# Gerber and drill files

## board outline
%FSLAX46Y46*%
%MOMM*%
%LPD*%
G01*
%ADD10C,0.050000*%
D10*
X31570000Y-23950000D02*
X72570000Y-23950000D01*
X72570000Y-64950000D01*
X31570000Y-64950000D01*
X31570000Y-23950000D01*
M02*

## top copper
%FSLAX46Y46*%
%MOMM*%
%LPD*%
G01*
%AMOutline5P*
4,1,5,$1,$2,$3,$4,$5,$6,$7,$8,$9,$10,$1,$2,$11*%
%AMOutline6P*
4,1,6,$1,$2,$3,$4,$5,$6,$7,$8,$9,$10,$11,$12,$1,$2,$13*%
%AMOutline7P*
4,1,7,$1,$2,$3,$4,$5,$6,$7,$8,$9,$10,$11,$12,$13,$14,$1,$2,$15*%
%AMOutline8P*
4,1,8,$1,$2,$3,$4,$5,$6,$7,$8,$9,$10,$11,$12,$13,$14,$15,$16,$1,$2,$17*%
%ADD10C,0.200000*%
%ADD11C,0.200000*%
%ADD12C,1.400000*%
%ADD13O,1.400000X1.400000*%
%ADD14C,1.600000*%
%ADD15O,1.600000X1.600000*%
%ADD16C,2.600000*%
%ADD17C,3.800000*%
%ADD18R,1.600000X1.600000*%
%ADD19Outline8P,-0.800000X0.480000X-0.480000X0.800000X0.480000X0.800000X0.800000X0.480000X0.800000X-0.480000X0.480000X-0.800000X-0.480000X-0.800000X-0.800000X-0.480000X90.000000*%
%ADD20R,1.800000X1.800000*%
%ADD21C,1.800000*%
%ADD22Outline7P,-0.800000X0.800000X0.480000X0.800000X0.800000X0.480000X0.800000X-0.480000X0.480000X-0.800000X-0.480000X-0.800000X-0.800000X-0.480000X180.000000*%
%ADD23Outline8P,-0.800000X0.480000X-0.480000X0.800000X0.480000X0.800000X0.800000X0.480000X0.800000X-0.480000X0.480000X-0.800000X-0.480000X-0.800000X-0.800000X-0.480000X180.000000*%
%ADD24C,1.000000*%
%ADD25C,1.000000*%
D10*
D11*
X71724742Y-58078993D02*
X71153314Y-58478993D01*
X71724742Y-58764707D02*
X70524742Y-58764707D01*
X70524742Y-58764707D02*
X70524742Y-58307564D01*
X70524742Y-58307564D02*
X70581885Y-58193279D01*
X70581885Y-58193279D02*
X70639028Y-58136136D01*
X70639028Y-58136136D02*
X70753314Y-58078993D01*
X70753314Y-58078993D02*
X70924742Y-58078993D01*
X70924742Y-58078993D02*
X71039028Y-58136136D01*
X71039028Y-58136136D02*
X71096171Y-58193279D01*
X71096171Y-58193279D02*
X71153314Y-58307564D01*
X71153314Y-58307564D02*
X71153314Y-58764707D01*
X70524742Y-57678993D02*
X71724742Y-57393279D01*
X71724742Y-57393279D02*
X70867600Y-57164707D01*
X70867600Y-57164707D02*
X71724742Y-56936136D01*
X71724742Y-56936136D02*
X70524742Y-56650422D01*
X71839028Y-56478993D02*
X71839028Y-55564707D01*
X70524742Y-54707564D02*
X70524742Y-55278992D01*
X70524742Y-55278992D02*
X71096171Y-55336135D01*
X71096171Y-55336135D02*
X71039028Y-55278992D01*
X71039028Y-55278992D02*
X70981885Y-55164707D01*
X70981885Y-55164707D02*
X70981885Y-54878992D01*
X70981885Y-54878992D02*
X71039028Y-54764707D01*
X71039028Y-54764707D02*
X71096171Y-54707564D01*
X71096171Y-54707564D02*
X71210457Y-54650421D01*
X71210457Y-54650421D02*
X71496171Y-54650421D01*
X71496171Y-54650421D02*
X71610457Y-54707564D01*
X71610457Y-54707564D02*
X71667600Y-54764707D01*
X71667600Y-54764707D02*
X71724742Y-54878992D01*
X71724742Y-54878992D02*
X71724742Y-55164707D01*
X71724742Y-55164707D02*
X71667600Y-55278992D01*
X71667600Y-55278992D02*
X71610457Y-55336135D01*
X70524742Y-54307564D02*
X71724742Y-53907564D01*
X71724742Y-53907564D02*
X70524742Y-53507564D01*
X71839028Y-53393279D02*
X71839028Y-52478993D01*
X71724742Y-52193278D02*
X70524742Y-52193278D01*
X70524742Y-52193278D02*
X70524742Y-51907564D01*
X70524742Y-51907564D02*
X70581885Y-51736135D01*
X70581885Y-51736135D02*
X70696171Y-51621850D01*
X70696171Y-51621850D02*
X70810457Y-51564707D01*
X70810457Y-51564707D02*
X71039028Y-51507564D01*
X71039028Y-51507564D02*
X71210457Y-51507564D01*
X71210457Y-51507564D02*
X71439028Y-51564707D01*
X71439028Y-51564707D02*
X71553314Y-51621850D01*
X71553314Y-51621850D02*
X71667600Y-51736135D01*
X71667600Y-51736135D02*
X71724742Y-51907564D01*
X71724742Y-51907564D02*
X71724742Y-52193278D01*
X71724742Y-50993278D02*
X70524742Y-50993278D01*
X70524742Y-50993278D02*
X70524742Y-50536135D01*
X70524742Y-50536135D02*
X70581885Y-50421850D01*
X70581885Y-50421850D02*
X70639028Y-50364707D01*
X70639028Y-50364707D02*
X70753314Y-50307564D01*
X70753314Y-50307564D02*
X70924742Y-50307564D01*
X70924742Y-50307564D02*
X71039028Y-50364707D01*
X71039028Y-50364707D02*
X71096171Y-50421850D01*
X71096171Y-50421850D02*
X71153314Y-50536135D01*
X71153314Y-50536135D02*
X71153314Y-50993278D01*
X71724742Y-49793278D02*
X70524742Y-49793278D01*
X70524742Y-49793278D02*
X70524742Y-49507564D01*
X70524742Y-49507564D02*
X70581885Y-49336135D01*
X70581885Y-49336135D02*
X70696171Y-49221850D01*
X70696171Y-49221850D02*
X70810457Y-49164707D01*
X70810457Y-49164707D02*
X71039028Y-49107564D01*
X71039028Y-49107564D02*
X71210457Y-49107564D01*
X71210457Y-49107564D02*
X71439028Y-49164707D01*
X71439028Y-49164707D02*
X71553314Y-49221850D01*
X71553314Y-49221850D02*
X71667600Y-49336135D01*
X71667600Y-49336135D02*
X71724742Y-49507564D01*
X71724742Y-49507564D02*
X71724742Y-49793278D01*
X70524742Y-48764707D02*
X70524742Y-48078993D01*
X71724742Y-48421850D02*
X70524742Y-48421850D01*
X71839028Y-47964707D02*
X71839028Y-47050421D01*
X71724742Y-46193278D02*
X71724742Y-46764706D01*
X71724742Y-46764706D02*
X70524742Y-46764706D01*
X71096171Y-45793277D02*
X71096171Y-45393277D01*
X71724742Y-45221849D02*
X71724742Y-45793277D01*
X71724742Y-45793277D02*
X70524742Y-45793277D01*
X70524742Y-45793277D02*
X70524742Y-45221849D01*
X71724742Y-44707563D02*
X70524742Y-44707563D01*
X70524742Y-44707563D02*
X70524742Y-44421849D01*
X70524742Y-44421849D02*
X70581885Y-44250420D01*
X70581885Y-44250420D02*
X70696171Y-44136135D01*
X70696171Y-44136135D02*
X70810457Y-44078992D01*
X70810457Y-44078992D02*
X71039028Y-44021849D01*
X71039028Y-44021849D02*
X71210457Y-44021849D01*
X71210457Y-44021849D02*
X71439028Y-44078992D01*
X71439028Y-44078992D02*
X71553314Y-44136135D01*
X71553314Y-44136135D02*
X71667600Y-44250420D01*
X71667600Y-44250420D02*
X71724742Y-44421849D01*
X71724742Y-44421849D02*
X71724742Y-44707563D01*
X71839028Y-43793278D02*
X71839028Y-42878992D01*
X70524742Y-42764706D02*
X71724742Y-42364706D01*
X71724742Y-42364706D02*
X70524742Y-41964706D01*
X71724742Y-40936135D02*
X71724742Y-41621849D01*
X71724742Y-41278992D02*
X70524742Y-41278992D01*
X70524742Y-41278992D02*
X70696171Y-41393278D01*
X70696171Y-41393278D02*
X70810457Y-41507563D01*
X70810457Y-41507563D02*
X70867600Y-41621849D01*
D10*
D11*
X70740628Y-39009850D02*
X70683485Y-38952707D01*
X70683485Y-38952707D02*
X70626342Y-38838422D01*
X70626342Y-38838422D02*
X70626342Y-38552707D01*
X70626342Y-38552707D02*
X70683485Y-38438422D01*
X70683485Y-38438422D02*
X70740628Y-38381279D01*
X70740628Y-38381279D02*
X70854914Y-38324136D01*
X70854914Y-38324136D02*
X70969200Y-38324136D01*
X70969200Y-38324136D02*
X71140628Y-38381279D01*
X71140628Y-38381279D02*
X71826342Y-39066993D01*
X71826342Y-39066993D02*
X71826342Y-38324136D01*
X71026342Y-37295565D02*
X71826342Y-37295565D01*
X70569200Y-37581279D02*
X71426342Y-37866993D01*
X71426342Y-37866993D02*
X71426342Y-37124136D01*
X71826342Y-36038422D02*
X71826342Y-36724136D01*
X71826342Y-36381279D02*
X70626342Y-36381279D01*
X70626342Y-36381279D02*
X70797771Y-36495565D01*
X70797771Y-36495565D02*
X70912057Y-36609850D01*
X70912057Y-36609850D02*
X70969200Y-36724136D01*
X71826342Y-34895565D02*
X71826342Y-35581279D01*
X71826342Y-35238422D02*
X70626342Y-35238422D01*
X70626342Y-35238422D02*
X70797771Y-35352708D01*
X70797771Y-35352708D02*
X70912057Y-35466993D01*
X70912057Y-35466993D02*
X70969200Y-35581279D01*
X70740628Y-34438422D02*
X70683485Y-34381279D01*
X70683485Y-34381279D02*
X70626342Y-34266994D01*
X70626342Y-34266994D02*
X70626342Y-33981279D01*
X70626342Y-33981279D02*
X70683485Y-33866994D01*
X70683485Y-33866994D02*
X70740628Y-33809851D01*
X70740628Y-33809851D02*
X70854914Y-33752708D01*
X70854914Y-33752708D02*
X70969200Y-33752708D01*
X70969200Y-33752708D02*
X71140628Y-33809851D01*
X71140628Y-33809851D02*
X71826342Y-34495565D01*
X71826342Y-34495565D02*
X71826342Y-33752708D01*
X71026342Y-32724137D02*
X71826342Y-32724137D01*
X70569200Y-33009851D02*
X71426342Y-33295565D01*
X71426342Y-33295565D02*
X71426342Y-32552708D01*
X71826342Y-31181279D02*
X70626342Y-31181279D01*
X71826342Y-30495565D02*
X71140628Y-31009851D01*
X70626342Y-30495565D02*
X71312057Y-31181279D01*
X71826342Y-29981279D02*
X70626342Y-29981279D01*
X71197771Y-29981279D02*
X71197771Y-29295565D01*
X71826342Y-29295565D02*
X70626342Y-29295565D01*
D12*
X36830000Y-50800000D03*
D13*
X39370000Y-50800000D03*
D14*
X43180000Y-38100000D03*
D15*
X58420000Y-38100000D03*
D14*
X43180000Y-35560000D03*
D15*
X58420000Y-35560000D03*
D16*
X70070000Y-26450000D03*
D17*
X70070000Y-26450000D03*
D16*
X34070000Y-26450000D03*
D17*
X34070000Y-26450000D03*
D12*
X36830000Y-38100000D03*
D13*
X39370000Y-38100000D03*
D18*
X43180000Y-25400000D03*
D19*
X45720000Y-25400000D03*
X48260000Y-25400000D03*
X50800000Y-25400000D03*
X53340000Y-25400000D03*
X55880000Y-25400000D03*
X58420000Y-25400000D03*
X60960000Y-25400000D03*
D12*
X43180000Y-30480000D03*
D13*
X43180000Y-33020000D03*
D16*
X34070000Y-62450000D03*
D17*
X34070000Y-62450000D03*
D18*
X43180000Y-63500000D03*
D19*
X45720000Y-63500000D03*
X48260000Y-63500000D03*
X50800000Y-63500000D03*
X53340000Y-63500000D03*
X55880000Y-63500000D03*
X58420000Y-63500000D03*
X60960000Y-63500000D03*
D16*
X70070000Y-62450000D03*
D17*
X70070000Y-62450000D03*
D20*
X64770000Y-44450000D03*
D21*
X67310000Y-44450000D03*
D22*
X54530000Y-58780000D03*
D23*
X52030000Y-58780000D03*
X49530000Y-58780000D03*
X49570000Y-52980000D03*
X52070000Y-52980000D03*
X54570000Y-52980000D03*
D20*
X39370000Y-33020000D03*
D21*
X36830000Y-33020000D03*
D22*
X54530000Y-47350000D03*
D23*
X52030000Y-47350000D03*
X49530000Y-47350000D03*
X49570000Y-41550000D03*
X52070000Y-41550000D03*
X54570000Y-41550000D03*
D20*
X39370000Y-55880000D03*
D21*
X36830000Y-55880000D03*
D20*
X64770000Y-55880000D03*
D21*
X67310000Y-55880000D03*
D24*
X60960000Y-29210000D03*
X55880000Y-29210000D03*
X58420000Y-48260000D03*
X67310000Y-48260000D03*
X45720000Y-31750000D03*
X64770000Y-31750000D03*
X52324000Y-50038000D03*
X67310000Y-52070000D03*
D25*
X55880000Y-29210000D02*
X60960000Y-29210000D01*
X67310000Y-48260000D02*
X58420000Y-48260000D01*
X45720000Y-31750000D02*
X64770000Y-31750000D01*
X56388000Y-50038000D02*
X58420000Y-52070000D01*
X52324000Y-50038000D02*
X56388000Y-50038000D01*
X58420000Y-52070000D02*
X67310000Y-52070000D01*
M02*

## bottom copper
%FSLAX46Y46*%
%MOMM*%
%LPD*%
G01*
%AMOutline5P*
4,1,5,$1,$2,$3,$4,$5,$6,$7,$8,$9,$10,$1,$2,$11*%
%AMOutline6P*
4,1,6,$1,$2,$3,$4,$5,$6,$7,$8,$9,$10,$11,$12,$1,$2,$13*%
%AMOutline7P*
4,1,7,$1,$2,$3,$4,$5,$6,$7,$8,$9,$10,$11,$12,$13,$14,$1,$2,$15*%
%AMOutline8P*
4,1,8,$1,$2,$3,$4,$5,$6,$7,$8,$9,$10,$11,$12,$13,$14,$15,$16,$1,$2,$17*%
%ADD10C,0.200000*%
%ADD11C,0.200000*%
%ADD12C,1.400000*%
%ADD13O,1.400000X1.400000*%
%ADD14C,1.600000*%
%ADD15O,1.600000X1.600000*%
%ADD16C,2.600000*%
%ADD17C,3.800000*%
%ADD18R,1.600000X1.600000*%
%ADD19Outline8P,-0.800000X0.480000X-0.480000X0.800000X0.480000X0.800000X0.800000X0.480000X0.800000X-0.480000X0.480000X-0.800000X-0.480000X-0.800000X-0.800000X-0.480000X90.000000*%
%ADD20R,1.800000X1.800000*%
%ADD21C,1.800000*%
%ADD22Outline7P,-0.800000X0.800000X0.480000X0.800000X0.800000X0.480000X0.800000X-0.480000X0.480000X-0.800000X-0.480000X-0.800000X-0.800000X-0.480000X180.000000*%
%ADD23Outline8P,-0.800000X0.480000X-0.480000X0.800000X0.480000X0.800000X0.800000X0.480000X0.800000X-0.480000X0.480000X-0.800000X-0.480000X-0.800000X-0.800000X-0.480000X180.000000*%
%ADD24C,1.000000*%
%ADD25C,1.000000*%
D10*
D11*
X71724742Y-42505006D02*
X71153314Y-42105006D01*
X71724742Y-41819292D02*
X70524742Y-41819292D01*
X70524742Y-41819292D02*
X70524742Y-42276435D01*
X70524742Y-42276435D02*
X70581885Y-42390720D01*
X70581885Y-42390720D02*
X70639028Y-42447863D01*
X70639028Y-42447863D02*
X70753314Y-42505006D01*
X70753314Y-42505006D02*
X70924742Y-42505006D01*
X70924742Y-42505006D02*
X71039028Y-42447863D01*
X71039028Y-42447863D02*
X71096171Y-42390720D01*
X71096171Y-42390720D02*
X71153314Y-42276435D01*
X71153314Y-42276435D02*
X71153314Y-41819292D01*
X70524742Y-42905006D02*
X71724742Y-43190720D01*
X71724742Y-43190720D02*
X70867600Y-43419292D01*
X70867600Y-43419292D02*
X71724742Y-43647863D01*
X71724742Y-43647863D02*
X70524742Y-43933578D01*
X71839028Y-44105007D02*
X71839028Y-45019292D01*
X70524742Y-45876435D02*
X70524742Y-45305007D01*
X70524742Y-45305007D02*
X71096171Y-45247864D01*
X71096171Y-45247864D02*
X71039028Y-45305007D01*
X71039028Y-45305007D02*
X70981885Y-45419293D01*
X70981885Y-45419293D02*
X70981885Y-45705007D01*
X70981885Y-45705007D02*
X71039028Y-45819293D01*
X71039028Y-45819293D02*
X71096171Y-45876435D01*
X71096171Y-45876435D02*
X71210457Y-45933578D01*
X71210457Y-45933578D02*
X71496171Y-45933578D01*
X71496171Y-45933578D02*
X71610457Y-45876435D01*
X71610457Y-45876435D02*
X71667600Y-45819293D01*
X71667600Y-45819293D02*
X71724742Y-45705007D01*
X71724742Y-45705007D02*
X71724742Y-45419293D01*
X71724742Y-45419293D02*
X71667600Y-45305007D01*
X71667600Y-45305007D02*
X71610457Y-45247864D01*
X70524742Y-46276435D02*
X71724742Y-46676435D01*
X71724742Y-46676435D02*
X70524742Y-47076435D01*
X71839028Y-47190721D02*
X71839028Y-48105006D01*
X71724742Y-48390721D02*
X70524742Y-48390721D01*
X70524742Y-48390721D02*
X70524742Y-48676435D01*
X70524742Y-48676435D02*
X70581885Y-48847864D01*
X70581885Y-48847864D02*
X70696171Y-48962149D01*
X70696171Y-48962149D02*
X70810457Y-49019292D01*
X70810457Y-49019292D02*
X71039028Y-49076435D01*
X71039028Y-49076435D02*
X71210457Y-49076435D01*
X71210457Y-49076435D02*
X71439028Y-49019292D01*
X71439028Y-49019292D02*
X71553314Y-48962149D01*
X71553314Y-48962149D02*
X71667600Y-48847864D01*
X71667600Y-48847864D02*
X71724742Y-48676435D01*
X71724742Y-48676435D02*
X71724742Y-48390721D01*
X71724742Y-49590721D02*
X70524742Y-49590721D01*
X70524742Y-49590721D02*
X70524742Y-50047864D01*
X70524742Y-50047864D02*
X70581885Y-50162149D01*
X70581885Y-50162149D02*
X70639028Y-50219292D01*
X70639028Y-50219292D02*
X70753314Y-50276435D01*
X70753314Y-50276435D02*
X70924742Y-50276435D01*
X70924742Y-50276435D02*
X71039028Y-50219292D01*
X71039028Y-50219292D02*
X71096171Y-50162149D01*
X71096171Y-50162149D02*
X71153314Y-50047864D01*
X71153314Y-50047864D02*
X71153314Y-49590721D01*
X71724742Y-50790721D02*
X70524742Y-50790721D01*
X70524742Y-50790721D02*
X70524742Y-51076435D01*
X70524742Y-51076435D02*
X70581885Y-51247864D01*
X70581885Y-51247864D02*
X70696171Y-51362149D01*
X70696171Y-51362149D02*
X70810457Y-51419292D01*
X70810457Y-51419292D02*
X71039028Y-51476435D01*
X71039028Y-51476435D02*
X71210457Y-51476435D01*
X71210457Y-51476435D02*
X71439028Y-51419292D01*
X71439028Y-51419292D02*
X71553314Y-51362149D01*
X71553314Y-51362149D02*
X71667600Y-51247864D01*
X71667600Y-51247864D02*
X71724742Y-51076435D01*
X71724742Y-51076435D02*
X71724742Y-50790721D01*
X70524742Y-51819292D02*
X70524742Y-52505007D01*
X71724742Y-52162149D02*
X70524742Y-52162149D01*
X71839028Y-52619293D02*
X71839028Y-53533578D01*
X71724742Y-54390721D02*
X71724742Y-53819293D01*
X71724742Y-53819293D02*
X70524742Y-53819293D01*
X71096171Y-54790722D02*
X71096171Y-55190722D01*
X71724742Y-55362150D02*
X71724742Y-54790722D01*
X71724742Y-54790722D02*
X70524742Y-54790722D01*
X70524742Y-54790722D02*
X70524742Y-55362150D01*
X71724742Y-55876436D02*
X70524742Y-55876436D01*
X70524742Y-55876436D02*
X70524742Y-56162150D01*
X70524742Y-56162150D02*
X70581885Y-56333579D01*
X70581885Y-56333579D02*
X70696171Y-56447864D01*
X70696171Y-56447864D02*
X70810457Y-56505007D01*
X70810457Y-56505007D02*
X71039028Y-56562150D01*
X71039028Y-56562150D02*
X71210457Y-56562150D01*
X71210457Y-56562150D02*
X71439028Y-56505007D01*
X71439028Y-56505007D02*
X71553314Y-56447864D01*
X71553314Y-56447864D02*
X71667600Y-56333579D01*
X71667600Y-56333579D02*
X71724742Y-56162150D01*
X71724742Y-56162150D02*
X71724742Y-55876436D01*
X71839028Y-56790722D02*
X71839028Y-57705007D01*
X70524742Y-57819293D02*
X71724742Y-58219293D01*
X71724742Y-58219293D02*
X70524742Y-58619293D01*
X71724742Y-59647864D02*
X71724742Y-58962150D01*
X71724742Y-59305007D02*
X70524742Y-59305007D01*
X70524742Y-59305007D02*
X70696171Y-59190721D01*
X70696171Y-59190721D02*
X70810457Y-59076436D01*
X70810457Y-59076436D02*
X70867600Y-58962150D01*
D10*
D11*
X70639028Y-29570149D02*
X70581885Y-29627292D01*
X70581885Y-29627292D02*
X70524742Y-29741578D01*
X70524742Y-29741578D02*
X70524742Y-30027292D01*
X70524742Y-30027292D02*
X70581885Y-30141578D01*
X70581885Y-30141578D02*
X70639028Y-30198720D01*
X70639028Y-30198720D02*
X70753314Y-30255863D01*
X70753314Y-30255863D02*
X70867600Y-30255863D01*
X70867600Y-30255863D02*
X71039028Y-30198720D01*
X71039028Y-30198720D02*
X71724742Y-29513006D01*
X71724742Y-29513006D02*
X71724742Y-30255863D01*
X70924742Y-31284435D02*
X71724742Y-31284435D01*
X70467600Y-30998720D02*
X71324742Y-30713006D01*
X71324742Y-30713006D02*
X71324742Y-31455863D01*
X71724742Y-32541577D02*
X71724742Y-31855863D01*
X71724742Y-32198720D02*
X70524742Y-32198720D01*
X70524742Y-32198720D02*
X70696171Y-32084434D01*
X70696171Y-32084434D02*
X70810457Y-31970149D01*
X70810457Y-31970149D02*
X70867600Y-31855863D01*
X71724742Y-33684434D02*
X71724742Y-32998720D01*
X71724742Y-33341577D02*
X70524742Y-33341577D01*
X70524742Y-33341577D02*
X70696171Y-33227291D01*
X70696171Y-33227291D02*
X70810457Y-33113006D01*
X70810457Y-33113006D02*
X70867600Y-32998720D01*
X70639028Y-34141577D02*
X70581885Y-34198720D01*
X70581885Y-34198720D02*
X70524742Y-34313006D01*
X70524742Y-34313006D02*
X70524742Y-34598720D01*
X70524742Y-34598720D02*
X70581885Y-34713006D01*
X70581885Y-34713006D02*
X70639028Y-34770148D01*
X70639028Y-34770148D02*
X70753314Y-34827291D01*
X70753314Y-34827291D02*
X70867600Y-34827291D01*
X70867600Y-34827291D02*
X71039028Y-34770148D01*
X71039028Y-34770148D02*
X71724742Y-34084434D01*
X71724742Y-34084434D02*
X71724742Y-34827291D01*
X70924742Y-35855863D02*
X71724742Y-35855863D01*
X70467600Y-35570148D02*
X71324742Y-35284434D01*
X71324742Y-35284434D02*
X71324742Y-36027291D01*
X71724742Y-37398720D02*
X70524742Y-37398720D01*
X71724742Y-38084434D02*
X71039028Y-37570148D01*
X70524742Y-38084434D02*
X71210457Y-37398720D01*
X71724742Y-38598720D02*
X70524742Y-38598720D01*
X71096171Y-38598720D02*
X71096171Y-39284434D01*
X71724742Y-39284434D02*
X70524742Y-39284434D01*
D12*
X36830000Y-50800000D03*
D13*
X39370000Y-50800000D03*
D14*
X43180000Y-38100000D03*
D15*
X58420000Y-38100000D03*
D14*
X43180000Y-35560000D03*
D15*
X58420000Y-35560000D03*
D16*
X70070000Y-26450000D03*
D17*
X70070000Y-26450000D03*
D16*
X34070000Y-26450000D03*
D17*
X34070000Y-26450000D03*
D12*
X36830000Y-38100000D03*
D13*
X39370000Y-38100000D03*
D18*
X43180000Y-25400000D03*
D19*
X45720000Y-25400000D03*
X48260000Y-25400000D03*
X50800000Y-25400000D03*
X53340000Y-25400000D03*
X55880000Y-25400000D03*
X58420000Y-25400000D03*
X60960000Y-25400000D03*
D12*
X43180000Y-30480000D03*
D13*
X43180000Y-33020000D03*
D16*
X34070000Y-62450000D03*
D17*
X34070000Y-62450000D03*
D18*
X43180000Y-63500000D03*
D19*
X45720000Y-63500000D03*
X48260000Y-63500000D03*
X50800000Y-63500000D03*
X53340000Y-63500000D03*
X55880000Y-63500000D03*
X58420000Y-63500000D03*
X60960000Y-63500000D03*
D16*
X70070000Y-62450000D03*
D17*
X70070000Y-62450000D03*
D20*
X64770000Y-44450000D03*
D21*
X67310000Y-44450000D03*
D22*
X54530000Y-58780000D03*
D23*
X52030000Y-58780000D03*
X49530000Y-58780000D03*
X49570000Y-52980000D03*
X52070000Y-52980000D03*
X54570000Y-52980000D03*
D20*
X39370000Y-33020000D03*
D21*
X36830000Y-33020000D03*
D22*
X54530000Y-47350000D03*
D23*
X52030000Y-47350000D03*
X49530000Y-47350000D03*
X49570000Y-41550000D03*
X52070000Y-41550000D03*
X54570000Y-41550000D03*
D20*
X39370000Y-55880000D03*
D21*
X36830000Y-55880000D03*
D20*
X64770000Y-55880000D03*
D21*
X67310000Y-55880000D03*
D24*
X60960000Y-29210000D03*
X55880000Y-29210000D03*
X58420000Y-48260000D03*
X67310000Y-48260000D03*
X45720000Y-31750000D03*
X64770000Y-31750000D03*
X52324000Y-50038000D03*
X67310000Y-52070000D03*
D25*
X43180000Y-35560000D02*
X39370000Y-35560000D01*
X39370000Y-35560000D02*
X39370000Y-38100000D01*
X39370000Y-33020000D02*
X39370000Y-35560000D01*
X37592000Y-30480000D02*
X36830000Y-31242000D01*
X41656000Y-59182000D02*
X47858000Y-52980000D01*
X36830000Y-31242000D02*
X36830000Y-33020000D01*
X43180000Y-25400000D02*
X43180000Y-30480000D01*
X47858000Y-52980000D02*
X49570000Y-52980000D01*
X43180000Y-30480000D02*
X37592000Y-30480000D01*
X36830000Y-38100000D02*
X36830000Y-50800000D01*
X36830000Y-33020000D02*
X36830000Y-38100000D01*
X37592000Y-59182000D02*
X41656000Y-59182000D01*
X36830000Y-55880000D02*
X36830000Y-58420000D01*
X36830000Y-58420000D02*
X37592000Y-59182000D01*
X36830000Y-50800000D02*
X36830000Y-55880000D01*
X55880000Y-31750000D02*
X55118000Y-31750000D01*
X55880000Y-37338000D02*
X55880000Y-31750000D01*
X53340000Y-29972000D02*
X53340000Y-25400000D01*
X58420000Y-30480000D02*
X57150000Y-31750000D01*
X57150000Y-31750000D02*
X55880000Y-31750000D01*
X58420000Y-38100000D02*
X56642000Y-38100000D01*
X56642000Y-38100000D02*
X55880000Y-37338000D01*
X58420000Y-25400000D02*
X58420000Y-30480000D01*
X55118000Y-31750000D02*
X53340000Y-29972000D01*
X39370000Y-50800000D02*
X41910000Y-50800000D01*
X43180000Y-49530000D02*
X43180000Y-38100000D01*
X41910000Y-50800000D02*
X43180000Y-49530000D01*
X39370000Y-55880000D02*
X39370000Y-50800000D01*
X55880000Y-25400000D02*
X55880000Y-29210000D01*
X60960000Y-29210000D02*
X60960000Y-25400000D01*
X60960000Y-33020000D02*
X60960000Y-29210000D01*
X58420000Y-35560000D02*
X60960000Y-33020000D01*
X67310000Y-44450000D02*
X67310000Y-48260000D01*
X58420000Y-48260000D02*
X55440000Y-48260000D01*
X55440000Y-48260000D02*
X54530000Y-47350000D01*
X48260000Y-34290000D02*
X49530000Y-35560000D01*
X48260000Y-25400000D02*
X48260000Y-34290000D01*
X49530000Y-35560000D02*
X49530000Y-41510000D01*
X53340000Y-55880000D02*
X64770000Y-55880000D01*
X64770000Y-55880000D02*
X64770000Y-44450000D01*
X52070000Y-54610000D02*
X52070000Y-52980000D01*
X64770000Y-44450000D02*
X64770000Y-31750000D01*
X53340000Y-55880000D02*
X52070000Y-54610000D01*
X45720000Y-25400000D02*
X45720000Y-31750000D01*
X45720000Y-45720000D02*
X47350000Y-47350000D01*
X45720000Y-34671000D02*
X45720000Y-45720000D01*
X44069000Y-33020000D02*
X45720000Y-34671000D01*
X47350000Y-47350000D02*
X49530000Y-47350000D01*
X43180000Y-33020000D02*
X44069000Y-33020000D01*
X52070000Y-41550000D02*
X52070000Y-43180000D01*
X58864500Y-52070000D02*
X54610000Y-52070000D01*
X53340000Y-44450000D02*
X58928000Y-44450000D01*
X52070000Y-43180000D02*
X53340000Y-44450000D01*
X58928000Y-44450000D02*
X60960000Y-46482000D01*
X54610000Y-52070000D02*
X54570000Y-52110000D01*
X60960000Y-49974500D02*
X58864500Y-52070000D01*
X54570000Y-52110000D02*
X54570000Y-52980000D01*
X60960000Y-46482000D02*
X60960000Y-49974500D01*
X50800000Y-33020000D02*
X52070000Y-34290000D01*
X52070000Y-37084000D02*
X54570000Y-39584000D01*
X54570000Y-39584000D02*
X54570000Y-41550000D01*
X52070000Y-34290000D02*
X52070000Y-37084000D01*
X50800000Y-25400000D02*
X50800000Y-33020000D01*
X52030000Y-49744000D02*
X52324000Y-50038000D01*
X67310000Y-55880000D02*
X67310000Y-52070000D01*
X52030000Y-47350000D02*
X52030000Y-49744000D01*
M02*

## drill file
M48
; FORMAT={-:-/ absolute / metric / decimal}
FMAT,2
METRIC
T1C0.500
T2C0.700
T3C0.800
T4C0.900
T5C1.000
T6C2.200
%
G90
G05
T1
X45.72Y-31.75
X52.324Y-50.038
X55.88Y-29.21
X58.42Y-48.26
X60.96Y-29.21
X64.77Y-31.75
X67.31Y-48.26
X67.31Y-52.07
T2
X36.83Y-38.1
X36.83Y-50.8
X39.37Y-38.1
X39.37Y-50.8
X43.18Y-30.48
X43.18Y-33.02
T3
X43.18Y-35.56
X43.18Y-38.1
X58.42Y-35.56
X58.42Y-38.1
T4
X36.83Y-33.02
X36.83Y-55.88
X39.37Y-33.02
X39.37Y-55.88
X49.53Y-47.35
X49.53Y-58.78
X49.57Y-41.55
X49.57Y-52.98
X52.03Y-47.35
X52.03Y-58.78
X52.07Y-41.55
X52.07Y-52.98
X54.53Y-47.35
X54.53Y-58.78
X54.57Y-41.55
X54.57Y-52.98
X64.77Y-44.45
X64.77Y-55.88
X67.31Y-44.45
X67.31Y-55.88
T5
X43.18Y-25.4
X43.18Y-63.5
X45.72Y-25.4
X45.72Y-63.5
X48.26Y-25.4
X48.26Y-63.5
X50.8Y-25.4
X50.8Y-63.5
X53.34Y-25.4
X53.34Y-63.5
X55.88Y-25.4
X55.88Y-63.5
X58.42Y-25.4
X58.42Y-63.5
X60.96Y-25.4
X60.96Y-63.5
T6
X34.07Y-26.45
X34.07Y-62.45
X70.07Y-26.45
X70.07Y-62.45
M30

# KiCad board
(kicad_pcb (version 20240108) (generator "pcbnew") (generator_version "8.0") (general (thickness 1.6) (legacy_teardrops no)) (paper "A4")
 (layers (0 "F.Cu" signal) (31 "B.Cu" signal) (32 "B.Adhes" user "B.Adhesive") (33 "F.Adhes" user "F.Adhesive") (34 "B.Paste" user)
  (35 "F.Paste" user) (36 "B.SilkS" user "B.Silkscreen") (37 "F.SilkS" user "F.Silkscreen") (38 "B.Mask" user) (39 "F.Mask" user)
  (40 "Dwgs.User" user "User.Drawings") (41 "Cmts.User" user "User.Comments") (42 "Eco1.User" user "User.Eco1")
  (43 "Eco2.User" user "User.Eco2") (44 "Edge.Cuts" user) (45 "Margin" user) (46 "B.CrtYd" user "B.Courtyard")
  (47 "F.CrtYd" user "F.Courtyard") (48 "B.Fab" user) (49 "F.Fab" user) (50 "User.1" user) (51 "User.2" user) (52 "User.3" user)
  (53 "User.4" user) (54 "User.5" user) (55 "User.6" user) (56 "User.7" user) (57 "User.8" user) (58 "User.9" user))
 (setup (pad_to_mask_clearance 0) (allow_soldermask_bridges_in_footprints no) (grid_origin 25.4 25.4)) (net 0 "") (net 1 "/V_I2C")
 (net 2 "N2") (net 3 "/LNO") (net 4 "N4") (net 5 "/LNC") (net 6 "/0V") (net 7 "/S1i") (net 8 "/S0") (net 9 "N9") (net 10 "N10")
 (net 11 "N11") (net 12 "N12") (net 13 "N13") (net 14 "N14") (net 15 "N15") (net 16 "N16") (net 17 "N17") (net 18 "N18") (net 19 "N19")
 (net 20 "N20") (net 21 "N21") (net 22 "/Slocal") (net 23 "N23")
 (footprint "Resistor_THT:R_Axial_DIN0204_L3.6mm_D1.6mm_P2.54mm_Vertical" (layer "F.Cu") (at 36.83 50.8)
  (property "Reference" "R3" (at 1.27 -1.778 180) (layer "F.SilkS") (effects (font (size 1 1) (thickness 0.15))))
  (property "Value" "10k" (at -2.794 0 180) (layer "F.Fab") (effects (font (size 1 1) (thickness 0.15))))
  (pad "1" thru_hole circle (at 0 0) (size 1.4 1.4) (drill 0.7) (layers "*.Cu" "*.Mask") (remove_unused_layers no) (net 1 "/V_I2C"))
  (pad "2" thru_hole oval (at 2.54 0) (size 1.4 1.4) (drill 0.7) (layers "*.Cu" "*.Mask") (remove_unused_layers no) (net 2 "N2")))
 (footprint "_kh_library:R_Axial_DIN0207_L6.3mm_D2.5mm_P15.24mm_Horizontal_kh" (layer "F.Cu") (at 43.18 38.1)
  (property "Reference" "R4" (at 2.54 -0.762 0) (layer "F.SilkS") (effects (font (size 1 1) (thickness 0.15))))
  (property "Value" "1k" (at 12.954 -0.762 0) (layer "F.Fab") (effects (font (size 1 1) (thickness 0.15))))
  (pad "1" thru_hole circle (at 0 0) (size 1.6 1.6) (drill 0.8) (layers "*.Cu" "*.Mask") (remove_unused_layers no) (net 2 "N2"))
  (pad "2" thru_hole oval (at 15.24 0) (size 1.6 1.6) (drill 0.8) (layers "*.Cu" "*.Mask") (remove_unused_layers no) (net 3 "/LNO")))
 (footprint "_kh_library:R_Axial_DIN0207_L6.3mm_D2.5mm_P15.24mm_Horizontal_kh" (layer "F.Cu") (at 43.18 35.56)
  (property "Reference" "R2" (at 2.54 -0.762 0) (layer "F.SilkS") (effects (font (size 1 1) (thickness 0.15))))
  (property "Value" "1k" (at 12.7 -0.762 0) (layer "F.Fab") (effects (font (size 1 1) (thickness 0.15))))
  (pad "1" thru_hole circle (at 0 0) (size 1.6 1.6) (drill 0.8) (layers "*.Cu" "*.Mask") (remove_unused_layers no) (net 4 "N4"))
  (pad "2" thru_hole oval (at 15.24 0) (size 1.6 1.6) (drill 0.8) (layers "*.Cu" "*.Mask") (remove_unused_layers no) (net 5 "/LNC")))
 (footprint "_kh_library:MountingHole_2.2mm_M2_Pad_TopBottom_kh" (layer "F.Cu") (at 70.07 26.45)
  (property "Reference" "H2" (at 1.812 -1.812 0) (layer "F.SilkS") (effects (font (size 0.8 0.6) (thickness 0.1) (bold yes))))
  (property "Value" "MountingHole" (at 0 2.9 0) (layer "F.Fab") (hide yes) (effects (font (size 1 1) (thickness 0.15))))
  (pad "1" thru_hole circle (at 0 0) (size 2.6 2.6) (drill 2.2) (layers "*.Cu" "*.Mask") (remove_unused_layers no))
  (pad "1" connect circle (at 0 0) (size 3.8 3.8) (layers "F.Cu" "F.Mask"))
  (pad "1" connect circle (at 0 0) (size 3.8 3.8) (layers "B.Cu" "B.Mask")))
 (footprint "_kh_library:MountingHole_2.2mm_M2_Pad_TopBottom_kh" (layer "F.Cu") (at 34.07 26.45)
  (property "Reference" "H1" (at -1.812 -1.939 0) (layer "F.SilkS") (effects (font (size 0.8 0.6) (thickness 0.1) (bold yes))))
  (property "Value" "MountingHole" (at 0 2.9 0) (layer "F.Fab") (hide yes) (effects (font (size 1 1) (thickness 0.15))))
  (pad "1" thru_hole circle (at 0 0) (size 2.6 2.6) (drill 2.2) (layers "*.Cu" "*.Mask") (remove_unused_layers no))
  (pad "1" connect circle (at 0 0) (size 3.8 3.8) (layers "F.Cu" "F.Mask"))
  (pad "1" connect circle (at 0 0) (size 3.8 3.8) (layers "B.Cu" "B.Mask")))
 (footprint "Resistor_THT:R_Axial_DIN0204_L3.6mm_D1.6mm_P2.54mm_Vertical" (layer "F.Cu") (at 36.83 38.1)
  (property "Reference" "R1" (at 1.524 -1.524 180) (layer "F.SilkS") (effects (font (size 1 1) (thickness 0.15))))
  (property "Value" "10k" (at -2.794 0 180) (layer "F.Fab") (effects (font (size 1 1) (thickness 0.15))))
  (pad "1" thru_hole circle (at 0 0) (size 1.4 1.4) (drill 0.7) (layers "*.Cu" "*.Mask") (remove_unused_layers no) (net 1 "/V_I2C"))
  (pad "2" thru_hole oval (at 2.54 0) (size 1.4 1.4) (drill 0.7) (layers "*.Cu" "*.Mask") (remove_unused_layers no) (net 4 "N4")))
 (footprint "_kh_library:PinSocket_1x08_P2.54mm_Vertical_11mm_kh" (layer "F.Cu") (at 43.18 25.4 90)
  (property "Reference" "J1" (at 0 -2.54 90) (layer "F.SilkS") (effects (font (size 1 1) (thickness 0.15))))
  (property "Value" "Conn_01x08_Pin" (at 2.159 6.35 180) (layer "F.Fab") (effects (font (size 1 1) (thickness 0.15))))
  (pad "1" thru_hole rect (at 0 0 90) (size 1.6 1.6) (drill 1) (layers "*.Cu" "*.Mask") (remove_unused_layers no) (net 1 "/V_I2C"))
  (pad "2" thru_hole roundrect (at 0 2.54 90) (size 1.6 1.6) (drill 1) (layers "*.Cu" "*.Mask") (remove_unused_layers no)
   (roundrect_rratio 0) (chamfer_ratio 0.2) (chamfer top_left top_right bottom_left bottom_right) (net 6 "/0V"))
  (pad "3" thru_hole roundrect (at 0 5.08 90) (size 1.6 1.6) (drill 1) (layers "*.Cu" "*.Mask") (remove_unused_layers no)
   (roundrect_rratio 0) (chamfer_ratio 0.2) (chamfer top_left top_right bottom_left bottom_right) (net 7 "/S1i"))
  (pad "4" thru_hole roundrect (at 0 7.62 90) (size 1.6 1.6) (drill 1) (layers "*.Cu" "*.Mask") (remove_unused_layers no)
   (roundrect_rratio 0) (chamfer_ratio 0.2) (chamfer top_left top_right bottom_left bottom_right) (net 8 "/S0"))
  (pad "5" thru_hole roundrect (at 0 10.16 90) (size 1.6 1.6) (drill 1) (layers "*.Cu" "*.Mask") (remove_unused_layers no)
   (roundrect_rratio 0) (chamfer_ratio 0.2) (chamfer top_left top_right bottom_left bottom_right) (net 3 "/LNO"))
  (pad "6" thru_hole roundrect (at 0 12.7 90) (size 1.6 1.6) (drill 1) (layers "*.Cu" "*.Mask") (remove_unused_layers no)
   (roundrect_rratio 0) (chamfer_ratio 0.2) (chamfer top_left top_right bottom_left bottom_right) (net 5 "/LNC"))
  (pad "7" thru_hole roundrect (at 0 15.24 90) (size 1.6 1.6) (drill 1) (layers "*.Cu" "*.Mask") (remove_unused_layers no)
   (roundrect_rratio 0) (chamfer_ratio 0.2) (chamfer top_left top_right bottom_left bottom_right) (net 3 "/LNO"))
  (pad "8" thru_hole roundrect (at 0 17.78 90) (size 1.6 1.6) (drill 1) (layers "*.Cu" "*.Mask") (remove_unused_layers no)
   (roundrect_rratio 0) (chamfer_ratio 0.2) (chamfer top_left top_right bottom_left bottom_right) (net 5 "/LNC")))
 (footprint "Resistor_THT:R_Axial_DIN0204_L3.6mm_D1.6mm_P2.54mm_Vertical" (layer "F.Cu") (at 43.18 30.48 -90)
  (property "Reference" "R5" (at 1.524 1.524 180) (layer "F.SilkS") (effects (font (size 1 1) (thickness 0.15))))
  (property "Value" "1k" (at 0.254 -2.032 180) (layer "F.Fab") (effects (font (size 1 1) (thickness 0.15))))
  (pad "1" thru_hole circle (at 0 0 270) (size 1.4 1.4) (drill 0.7) (layers "*.Cu" "*.Mask") (remove_unused_layers no) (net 1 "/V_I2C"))
  (pad "2" thru_hole oval (at 2.54 0 270) (size 1.4 1.4) (drill 0.7) (layers "*.Cu" "*.Mask") (remove_unused_layers no) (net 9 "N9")))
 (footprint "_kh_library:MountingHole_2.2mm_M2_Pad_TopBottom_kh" (layer "F.Cu") (at 34.07 62.45)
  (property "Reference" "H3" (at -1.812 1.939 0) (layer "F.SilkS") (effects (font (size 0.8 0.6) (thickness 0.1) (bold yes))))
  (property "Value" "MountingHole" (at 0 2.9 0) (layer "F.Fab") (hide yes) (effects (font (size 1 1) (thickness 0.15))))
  (pad "1" thru_hole circle (at 0 0) (size 2.6 2.6) (drill 2.2) (layers "*.Cu" "*.Mask") (remove_unused_layers no))
  (pad "1" connect circle (at 0 0) (size 3.8 3.8) (layers "F.Cu" "F.Mask"))
  (pad "1" connect circle (at 0 0) (size 3.8 3.8) (layers "B.Cu" "B.Mask")))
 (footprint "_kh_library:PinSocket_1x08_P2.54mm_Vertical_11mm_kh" (layer "F.Cu") (at 43.18 63.5 90)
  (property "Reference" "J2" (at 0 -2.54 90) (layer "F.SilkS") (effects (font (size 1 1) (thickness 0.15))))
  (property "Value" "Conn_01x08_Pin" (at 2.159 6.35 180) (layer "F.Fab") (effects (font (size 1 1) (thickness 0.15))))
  (pad "1" thru_hole rect (at 0 0 90) (size 1.6 1.6) (drill 1) (layers "*.Cu" "*.Mask") (remove_unused_layers no) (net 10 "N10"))
  (pad "2" thru_hole roundrect (at 0 2.54 90) (size 1.6 1.6) (drill 1) (layers "*.Cu" "*.Mask") (remove_unused_layers no)
   (roundrect_rratio 0) (chamfer_ratio 0.2) (chamfer top_left top_right bottom_left bottom_right) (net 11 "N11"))
  (pad "3" thru_hole roundrect (at 0 5.08 90) (size 1.6 1.6) (drill 1) (layers "*.Cu" "*.Mask") (remove_unused_layers no)
   (roundrect_rratio 0) (chamfer_ratio 0.2) (chamfer top_left top_right bottom_left bottom_right) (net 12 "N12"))
  (pad "4" thru_hole roundrect (at 0 7.62 90) (size 1.6 1.6) (drill 1) (layers "*.Cu" "*.Mask") (remove_unused_layers no)
   (roundrect_rratio 0) (chamfer_ratio 0.2) (chamfer top_left top_right bottom_left bottom_right) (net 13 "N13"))
  (pad "5" thru_hole roundrect (at 0 10.16 90) (size 1.6 1.6) (drill 1) (layers "*.Cu" "*.Mask") (remove_unused_layers no)
   (roundrect_rratio 0) (chamfer_ratio 0.2) (chamfer top_left top_right bottom_left bottom_right) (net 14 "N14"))
  (pad "6" thru_hole roundrect (at 0 12.7 90) (size 1.6 1.6) (drill 1) (layers "*.Cu" "*.Mask") (remove_unused_layers no)
   (roundrect_rratio 0) (chamfer_ratio 0.2) (chamfer top_left top_right bottom_left bottom_right) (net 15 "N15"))
  (pad "7" thru_hole roundrect (at 0 15.24 90) (size 1.6 1.6) (drill 1) (layers "*.Cu" "*.Mask") (remove_unused_layers no)
   (roundrect_rratio 0) (chamfer_ratio 0.2) (chamfer top_left top_right bottom_left bottom_right) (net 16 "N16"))
  (pad "8" thru_hole roundrect (at 0 17.78 90) (size 1.6 1.6) (drill 1) (layers "*.Cu" "*.Mask") (remove_unused_layers no)
   (roundrect_rratio 0) (chamfer_ratio 0.2) (chamfer top_left top_right bottom_left bottom_right) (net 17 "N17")))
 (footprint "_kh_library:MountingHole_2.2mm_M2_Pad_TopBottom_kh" (layer "F.Cu") (at 70.07 62.45)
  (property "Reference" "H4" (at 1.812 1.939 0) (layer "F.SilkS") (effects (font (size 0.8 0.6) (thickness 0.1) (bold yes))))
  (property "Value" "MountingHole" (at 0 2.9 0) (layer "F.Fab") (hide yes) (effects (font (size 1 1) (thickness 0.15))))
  (pad "1" thru_hole circle (at 0 0) (size 2.6 2.6) (drill 2.2) (layers "*.Cu" "*.Mask") (remove_unused_layers no))
  (pad "1" connect circle (at 0 0) (size 3.8 3.8) (layers "F.Cu" "F.Mask"))
  (pad "1" connect circle (at 0 0) (size 3.8 3.8) (layers "B.Cu" "B.Mask")))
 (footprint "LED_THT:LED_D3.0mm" (layer "B.Cu") (at 64.77 44.45)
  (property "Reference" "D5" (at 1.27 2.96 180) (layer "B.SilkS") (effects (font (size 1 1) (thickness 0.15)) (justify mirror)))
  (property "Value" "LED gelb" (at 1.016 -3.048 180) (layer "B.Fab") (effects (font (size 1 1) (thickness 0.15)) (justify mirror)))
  (pad "1" thru_hole rect (at 0 0) (size 1.8 1.8) (drill 0.9) (layers "*.Cu" "*.Mask") (remove_unused_layers no) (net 6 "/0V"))
  (pad "2" thru_hole circle (at 2.54 0) (size 1.8 1.8) (drill 0.9) (layers "*.Cu" "*.Mask") (remove_unused_layers no) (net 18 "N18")))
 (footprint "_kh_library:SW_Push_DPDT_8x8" (layer "B.Cu") (at 54.57 58.78 180)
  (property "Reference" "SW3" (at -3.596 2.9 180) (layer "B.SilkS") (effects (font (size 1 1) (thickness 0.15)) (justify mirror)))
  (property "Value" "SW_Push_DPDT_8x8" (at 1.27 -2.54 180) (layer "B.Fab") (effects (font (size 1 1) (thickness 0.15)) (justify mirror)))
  (pad "1" thru_hole roundrect (at 0.04 0 180) (size 1.6 1.6) (drill 0.9) (layers "*.Cu" "*.Mask") (remove_unused_layers no)
   (roundrect_rratio 0) (chamfer_ratio 0.2) (chamfer top_right bottom_left bottom_right) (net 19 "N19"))
  (pad "2" thru_hole roundrect (at 2.54 0 180) (size 1.6 1.6) (drill 0.9) (layers "*.Cu" "*.Mask") (remove_unused_layers no)
   (roundrect_rratio 0) (chamfer_ratio 0.2) (chamfer top_left top_right bottom_left bottom_right) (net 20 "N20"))
  (pad "3" thru_hole roundrect (at 5.04 0 180) (size 1.6 1.6) (drill 0.9) (layers "*.Cu" "*.Mask") (remove_unused_layers no)
   (roundrect_rratio 0) (chamfer_ratio 0.2) (chamfer top_left top_right bottom_left bottom_right) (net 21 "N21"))
  (pad "4" thru_hole roundrect (at 5 5.8 180) (size 1.6 1.6) (drill 0.9) (layers "*.Cu" "*.Mask") (remove_unused_layers no)
   (roundrect_rratio 0) (chamfer_ratio 0.2) (chamfer top_left top_right bottom_left bottom_right) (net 1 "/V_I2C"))
  (pad "5" thru_hole roundrect (at 2.5 5.8 180) (size 1.6 1.6) (drill 0.9) (layers "*.Cu" "*.Mask") (remove_unused_layers no)
   (roundrect_rratio 0) (chamfer_ratio 0.2) (chamfer top_left top_right bottom_left bottom_right) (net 6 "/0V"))
  (pad "6" thru_hole roundrect (at 0 5.8 180) (size 1.6 1.6) (drill 0.9) (layers "*.Cu" "*.Mask") (remove_unused_layers no)
   (roundrect_rratio 0) (chamfer_ratio 0.2) (chamfer top_left top_right bottom_left bottom_right) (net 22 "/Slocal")))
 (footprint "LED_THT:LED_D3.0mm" (layer "B.Cu") (at 39.37 33.02 180)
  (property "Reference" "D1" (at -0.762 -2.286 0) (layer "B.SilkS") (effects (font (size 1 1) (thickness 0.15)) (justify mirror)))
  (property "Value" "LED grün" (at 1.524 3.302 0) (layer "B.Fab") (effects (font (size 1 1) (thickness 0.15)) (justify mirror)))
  (pad "1" thru_hole rect (at 0 0 180) (size 1.8 1.8) (drill 0.9) (layers "*.Cu" "*.Mask") (remove_unused_layers no) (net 4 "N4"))
  (pad "2" thru_hole circle (at 2.54 0 180) (size 1.8 1.8) (drill 0.9) (layers "*.Cu" "*.Mask") (remove_unused_layers no) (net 1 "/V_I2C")))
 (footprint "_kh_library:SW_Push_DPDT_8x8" (layer "B.Cu") (at 54.57 47.35 180)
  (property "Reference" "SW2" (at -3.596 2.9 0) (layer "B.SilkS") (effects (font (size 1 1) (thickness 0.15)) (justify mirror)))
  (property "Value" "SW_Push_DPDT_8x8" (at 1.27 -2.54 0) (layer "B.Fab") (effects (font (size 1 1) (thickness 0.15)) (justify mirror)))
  (pad "1" thru_hole roundrect (at 0.04 0 180) (size 1.6 1.6) (drill 0.9) (layers "*.Cu" "*.Mask") (remove_unused_layers no)
   (roundrect_rratio 0) (chamfer_ratio 0.2) (chamfer top_right bottom_left bottom_right) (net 18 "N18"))
  (pad "2" thru_hole roundrect (at 2.54 0 180) (size 1.6 1.6) (drill 0.9) (layers "*.Cu" "*.Mask") (remove_unused_layers no)
   (roundrect_rratio 0) (chamfer_ratio 0.2) (chamfer top_left top_right bottom_left bottom_right) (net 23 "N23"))
  (pad "3" thru_hole roundrect (at 5.04 0 180) (size 1.6 1.6) (drill 0.9) (layers "*.Cu" "*.Mask") (remove_unused_layers no)
   (roundrect_rratio 0) (chamfer_ratio 0.2) (chamfer top_left top_right bottom_left bottom_right) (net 9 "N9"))
  (pad "4" thru_hole roundrect (at 5 5.8 180) (size 1.6 1.6) (drill 0.9) (layers "*.Cu" "*.Mask") (remove_unused_layers no)
   (roundrect_rratio 0) (chamfer_ratio 0.2) (chamfer top_left top_right bottom_left bottom_right) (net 7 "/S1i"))
  (pad "5" thru_hole roundrect (at 2.5 5.8 180) (size 1.6 1.6) (drill 0.9) (layers "*.Cu" "*.Mask") (remove_unused_layers no)
   (roundrect_rratio 0) (chamfer_ratio 0.2) (chamfer top_left top_right bottom_left bottom_right) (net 22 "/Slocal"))
  (pad "6" thru_hole roundrect (at 0 5.8 180) (size 1.6 1.6) (drill 0.9) (layers "*.Cu" "*.Mask") (remove_unused_layers no)
   (roundrect_rratio 0) (chamfer_ratio 0.2) (chamfer top_left top_right bottom_left bottom_right) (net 8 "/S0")))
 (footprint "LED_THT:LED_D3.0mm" (layer "B.Cu") (at 39.37 55.88 180)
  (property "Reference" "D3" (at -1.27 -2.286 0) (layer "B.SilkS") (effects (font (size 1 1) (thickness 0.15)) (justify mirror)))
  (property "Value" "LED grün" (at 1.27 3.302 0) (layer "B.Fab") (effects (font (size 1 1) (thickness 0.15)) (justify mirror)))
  (pad "1" thru_hole rect (at 0 0 180) (size 1.8 1.8) (drill 0.9) (layers "*.Cu" "*.Mask") (remove_unused_layers no) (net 2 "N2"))
  (pad "2" thru_hole circle (at 2.54 0 180) (size 1.8 1.8) (drill 0.9) (layers "*.Cu" "*.Mask") (remove_unused_layers no) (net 1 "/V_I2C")))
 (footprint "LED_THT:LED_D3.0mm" (layer "B.Cu") (at 64.77 55.88)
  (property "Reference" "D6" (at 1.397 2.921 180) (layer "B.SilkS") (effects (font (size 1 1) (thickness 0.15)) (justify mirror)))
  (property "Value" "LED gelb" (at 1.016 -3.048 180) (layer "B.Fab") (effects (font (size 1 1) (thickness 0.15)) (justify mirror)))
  (pad "1" thru_hole rect (at 0 0) (size 1.8 1.8) (drill 0.9) (layers "*.Cu" "*.Mask") (remove_unused_layers no) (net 6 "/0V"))
  (pad "2" thru_hole circle (at 2.54 0) (size 1.8 1.8) (drill 0.9) (layers "*.Cu" "*.Mask") (remove_unused_layers no) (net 23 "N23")))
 (gr_rect (start 31.57 23.95) (end 72.57 64.95) (stroke (width 0.05) (type default)) (fill none) (layer "Edge.Cuts"))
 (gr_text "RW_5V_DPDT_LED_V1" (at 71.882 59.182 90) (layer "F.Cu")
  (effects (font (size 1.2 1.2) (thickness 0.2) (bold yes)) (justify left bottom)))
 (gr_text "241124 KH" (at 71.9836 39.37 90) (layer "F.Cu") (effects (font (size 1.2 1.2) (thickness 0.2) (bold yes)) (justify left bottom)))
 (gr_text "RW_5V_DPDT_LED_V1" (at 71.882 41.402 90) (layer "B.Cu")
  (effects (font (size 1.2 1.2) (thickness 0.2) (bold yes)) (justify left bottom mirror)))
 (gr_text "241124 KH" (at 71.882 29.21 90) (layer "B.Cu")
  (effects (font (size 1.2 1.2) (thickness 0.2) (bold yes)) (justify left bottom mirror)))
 (segment (start 43.18 35.56) (end 39.37 35.56) (width 1) (layer "B.Cu") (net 4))
 (segment (start 39.37 35.56) (end 39.37 38.1) (width 1) (layer "B.Cu") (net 4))
 (segment (start 39.37 33.02) (end 39.37 35.56) (width 1) (layer "B.Cu") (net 4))
 (segment (start 37.592 30.48) (end 36.83 31.242) (width 1) (layer "B.Cu") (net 1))
 (segment (start 41.656 59.182) (end 47.858 52.98) (width 1) (layer "B.Cu") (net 1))
 (segment (start 36.83 31.242) (end 36.83 33.02) (width 1) (layer "B.Cu") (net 1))
 (segment (start 43.18 25.4) (end 43.18 30.48) (width 1) (layer "B.Cu") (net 1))
 (segment (start 47.858 52.98) (end 49.57 52.98) (width 1) (layer "B.Cu") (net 1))
 (segment (start 43.18 30.48) (end 37.592 30.48) (width 1) (layer "B.Cu") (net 1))
 (segment (start 36.83 38.1) (end 36.83 50.8) (width 1) (layer "B.Cu") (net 1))
 (segment (start 36.83 33.02) (end 36.83 38.1) (width 1) (layer "B.Cu") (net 1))
 (segment (start 37.592 59.182) (end 41.656 59.182) (width 1) (layer "B.Cu") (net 1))
 (segment (start 36.83 55.88) (end 36.83 58.42) (width 1) (layer "B.Cu") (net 1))
 (segment (start 36.83 58.42) (end 37.592 59.182) (width 1) (layer "B.Cu") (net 1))
 (segment (start 36.83 50.8) (end 36.83 55.88) (width 1) (layer "B.Cu") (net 1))
 (segment (start 55.88 31.75) (end 55.118 31.75) (width 1) (layer "B.Cu") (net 3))
 (segment (start 55.88 37.338) (end 55.88 31.75) (width 1) (layer "B.Cu") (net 3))
 (segment (start 53.34 29.972) (end 53.34 25.4) (width 1) (layer "B.Cu") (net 3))
 (segment (start 58.42 30.48) (end 57.15 31.75) (width 1) (layer "B.Cu") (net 3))
 (segment (start 57.15 31.75) (end 55.88 31.75) (width 1) (layer "B.Cu") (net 3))
 (segment (start 58.42 38.1) (end 56.642 38.1) (width 1) (layer "B.Cu") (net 3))
 (segment (start 56.642 38.1) (end 55.88 37.338) (width 1) (layer "B.Cu") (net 3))
 (segment (start 58.42 25.4) (end 58.42 30.48) (width 1) (layer "B.Cu") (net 3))
 (segment (start 55.118 31.75) (end 53.34 29.972) (width 1) (layer "B.Cu") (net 3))
 (segment (start 39.37 50.8) (end 41.91 50.8) (width 1) (layer "B.Cu") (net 2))
 (segment (start 43.18 49.53) (end 43.18 38.1) (width 1) (layer "B.Cu") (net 2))
 (segment (start 41.91 50.8) (end 43.18 49.53) (width 1) (layer "B.Cu") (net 2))
 (segment (start 39.37 55.88) (end 39.37 50.8) (width 1) (layer "B.Cu") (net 2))
 (segment (start 55.88 29.21) (end 60.96 29.21) (width 1) (layer "F.Cu") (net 5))
 (via (at 60.96 29.21) (size 1) (drill 0.5) (layers "F.Cu" "B.Cu") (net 5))
 (via (at 55.88 29.21) (size 1) (drill 0.5) (layers "F.Cu" "B.Cu") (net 5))
 (segment (start 55.88 25.4) (end 55.88 29.21) (width 1) (layer "B.Cu") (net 5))
 (segment (start 60.96 29.21) (end 60.96 25.4) (width 1) (layer "B.Cu") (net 5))
 (segment (start 60.96 33.02) (end 60.96 29.21) (width 1) (layer "B.Cu") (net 5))
 (segment (start 58.42 35.56) (end 60.96 33.02) (width 1) (layer "B.Cu") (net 5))
 (segment (start 67.31 48.26) (end 58.42 48.26) (width 1) (layer "F.Cu") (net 18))
 (via (at 58.42 48.26) (size 1) (drill 0.5) (layers "F.Cu" "B.Cu") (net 18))
 (via (at 67.31 48.26) (size 1) (drill 0.5) (layers "F.Cu" "B.Cu") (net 18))
 (segment (start 67.31 44.45) (end 67.31 48.26) (width 1) (layer "B.Cu") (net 18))
 (segment (start 58.42 48.26) (end 55.44 48.26) (width 1) (layer "B.Cu") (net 18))
 (segment (start 55.44 48.26) (end 54.53 47.35) (width 1) (layer "B.Cu") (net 18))
 (segment (start 48.26 34.29) (end 49.53 35.56) (width 1) (layer "B.Cu") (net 7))
 (segment (start 48.26 25.4) (end 48.26 34.29) (width 1) (layer "B.Cu") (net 7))
 (segment (start 49.53 35.56) (end 49.53 41.51) (width 1) (layer "B.Cu") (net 7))
 (segment (start 45.72 31.75) (end 64.77 31.75) (width 1) (layer "F.Cu") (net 6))
 (via (at 45.72 31.75) (size 1) (drill 0.5) (layers "F.Cu" "B.Cu") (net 6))
 (via (at 64.77 31.75) (size 1) (drill 0.5) (layers "F.Cu" "B.Cu") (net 6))
 (segment (start 53.34 55.88) (end 64.77 55.88) (width 1) (layer "B.Cu") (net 6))
 (segment (start 64.77 55.88) (end 64.77 44.45) (width 1) (layer "B.Cu") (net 6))
 (segment (start 52.07 54.61) (end 52.07 52.98) (width 1) (layer "B.Cu") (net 6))
 (segment (start 64.77 44.45) (end 64.77 31.75) (width 1) (layer "B.Cu") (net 6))
 (segment (start 53.34 55.88) (end 52.07 54.61) (width 1) (layer "B.Cu") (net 6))
 (segment (start 45.72 25.4) (end 45.72 31.75) (width 1) (layer "B.Cu") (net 6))
 (segment (start 45.72 45.72) (end 47.35 47.35) (width 1) (layer "B.Cu") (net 9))
 (segment (start 45.72 34.671) (end 45.72 45.72) (width 1) (layer "B.Cu") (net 9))
 (segment (start 44.069 33.02) (end 45.72 34.671) (width 1) (layer "B.Cu") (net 9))
 (segment (start 47.35 47.35) (end 49.53 47.35) (width 1) (layer "B.Cu") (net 9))
 (segment (start 43.18 33.02) (end 44.069 33.02) (width 1) (layer "B.Cu") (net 9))
 (segment (start 52.07 41.55) (end 52.07 43.18) (width 1) (layer "B.Cu") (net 22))
 (segment (start 58.8645 52.07) (end 54.61 52.07) (width 1) (layer "B.Cu") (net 22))
 (segment (start 53.34 44.45) (end 58.928 44.45) (width 1) (layer "B.Cu") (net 22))
 (segment (start 52.07 43.18) (end 53.34 44.45) (width 1) (layer "B.Cu") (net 22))
 (segment (start 58.928 44.45) (end 60.96 46.482) (width 1) (layer "B.Cu") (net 22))
 (segment (start 54.61 52.07) (end 54.57 52.11) (width 1) (layer "B.Cu") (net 22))
 (segment (start 60.96 49.9745) (end 58.8645 52.07) (width 1) (layer "B.Cu") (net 22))
 (segment (start 54.57 52.11) (end 54.57 52.98) (width 1) (layer "B.Cu") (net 22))
 (segment (start 60.96 46.482) (end 60.96 49.9745) (width 1) (layer "B.Cu") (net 22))
 (segment (start 50.8 33.02) (end 52.07 34.29) (width 1) (layer "B.Cu") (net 8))
 (segment (start 52.07 37.084) (end 54.57 39.584) (width 1) (layer "B.Cu") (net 8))
 (segment (start 54.57 39.584) (end 54.57 41.55) (width 1) (layer "B.Cu") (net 8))
 (segment (start 52.07 34.29) (end 52.07 37.084) (width 1) (layer "B.Cu") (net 8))
 (segment (start 50.8 25.4) (end 50.8 33.02) (width 1) (layer "B.Cu") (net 8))
 (segment (start 56.388 50.038) (end 58.42 52.07) (width 1) (layer "F.Cu") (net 23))
 (segment (start 52.324 50.038) (end 56.388 50.038) (width 1) (layer "F.Cu") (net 23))
 (segment (start 58.42 52.07) (end 67.31 52.07) (width 1) (layer "F.Cu") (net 23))
 (via (at 52.324 50.038) (size 1) (drill 0.5) (layers "F.Cu" "B.Cu") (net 23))
 (via (at 67.31 52.07) (size 1) (drill 0.5) (layers "F.Cu" "B.Cu") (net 23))
 (segment (start 52.03 49.744) (end 52.324 50.038) (width 1) (layer "B.Cu") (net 23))
 (segment (start 67.31 55.88) (end 67.31 52.07) (width 1) (layer "B.Cu") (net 23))
 (segment (start 52.03 47.35) (end 52.03 49.744) (width 1) (layer "B.Cu") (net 23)))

